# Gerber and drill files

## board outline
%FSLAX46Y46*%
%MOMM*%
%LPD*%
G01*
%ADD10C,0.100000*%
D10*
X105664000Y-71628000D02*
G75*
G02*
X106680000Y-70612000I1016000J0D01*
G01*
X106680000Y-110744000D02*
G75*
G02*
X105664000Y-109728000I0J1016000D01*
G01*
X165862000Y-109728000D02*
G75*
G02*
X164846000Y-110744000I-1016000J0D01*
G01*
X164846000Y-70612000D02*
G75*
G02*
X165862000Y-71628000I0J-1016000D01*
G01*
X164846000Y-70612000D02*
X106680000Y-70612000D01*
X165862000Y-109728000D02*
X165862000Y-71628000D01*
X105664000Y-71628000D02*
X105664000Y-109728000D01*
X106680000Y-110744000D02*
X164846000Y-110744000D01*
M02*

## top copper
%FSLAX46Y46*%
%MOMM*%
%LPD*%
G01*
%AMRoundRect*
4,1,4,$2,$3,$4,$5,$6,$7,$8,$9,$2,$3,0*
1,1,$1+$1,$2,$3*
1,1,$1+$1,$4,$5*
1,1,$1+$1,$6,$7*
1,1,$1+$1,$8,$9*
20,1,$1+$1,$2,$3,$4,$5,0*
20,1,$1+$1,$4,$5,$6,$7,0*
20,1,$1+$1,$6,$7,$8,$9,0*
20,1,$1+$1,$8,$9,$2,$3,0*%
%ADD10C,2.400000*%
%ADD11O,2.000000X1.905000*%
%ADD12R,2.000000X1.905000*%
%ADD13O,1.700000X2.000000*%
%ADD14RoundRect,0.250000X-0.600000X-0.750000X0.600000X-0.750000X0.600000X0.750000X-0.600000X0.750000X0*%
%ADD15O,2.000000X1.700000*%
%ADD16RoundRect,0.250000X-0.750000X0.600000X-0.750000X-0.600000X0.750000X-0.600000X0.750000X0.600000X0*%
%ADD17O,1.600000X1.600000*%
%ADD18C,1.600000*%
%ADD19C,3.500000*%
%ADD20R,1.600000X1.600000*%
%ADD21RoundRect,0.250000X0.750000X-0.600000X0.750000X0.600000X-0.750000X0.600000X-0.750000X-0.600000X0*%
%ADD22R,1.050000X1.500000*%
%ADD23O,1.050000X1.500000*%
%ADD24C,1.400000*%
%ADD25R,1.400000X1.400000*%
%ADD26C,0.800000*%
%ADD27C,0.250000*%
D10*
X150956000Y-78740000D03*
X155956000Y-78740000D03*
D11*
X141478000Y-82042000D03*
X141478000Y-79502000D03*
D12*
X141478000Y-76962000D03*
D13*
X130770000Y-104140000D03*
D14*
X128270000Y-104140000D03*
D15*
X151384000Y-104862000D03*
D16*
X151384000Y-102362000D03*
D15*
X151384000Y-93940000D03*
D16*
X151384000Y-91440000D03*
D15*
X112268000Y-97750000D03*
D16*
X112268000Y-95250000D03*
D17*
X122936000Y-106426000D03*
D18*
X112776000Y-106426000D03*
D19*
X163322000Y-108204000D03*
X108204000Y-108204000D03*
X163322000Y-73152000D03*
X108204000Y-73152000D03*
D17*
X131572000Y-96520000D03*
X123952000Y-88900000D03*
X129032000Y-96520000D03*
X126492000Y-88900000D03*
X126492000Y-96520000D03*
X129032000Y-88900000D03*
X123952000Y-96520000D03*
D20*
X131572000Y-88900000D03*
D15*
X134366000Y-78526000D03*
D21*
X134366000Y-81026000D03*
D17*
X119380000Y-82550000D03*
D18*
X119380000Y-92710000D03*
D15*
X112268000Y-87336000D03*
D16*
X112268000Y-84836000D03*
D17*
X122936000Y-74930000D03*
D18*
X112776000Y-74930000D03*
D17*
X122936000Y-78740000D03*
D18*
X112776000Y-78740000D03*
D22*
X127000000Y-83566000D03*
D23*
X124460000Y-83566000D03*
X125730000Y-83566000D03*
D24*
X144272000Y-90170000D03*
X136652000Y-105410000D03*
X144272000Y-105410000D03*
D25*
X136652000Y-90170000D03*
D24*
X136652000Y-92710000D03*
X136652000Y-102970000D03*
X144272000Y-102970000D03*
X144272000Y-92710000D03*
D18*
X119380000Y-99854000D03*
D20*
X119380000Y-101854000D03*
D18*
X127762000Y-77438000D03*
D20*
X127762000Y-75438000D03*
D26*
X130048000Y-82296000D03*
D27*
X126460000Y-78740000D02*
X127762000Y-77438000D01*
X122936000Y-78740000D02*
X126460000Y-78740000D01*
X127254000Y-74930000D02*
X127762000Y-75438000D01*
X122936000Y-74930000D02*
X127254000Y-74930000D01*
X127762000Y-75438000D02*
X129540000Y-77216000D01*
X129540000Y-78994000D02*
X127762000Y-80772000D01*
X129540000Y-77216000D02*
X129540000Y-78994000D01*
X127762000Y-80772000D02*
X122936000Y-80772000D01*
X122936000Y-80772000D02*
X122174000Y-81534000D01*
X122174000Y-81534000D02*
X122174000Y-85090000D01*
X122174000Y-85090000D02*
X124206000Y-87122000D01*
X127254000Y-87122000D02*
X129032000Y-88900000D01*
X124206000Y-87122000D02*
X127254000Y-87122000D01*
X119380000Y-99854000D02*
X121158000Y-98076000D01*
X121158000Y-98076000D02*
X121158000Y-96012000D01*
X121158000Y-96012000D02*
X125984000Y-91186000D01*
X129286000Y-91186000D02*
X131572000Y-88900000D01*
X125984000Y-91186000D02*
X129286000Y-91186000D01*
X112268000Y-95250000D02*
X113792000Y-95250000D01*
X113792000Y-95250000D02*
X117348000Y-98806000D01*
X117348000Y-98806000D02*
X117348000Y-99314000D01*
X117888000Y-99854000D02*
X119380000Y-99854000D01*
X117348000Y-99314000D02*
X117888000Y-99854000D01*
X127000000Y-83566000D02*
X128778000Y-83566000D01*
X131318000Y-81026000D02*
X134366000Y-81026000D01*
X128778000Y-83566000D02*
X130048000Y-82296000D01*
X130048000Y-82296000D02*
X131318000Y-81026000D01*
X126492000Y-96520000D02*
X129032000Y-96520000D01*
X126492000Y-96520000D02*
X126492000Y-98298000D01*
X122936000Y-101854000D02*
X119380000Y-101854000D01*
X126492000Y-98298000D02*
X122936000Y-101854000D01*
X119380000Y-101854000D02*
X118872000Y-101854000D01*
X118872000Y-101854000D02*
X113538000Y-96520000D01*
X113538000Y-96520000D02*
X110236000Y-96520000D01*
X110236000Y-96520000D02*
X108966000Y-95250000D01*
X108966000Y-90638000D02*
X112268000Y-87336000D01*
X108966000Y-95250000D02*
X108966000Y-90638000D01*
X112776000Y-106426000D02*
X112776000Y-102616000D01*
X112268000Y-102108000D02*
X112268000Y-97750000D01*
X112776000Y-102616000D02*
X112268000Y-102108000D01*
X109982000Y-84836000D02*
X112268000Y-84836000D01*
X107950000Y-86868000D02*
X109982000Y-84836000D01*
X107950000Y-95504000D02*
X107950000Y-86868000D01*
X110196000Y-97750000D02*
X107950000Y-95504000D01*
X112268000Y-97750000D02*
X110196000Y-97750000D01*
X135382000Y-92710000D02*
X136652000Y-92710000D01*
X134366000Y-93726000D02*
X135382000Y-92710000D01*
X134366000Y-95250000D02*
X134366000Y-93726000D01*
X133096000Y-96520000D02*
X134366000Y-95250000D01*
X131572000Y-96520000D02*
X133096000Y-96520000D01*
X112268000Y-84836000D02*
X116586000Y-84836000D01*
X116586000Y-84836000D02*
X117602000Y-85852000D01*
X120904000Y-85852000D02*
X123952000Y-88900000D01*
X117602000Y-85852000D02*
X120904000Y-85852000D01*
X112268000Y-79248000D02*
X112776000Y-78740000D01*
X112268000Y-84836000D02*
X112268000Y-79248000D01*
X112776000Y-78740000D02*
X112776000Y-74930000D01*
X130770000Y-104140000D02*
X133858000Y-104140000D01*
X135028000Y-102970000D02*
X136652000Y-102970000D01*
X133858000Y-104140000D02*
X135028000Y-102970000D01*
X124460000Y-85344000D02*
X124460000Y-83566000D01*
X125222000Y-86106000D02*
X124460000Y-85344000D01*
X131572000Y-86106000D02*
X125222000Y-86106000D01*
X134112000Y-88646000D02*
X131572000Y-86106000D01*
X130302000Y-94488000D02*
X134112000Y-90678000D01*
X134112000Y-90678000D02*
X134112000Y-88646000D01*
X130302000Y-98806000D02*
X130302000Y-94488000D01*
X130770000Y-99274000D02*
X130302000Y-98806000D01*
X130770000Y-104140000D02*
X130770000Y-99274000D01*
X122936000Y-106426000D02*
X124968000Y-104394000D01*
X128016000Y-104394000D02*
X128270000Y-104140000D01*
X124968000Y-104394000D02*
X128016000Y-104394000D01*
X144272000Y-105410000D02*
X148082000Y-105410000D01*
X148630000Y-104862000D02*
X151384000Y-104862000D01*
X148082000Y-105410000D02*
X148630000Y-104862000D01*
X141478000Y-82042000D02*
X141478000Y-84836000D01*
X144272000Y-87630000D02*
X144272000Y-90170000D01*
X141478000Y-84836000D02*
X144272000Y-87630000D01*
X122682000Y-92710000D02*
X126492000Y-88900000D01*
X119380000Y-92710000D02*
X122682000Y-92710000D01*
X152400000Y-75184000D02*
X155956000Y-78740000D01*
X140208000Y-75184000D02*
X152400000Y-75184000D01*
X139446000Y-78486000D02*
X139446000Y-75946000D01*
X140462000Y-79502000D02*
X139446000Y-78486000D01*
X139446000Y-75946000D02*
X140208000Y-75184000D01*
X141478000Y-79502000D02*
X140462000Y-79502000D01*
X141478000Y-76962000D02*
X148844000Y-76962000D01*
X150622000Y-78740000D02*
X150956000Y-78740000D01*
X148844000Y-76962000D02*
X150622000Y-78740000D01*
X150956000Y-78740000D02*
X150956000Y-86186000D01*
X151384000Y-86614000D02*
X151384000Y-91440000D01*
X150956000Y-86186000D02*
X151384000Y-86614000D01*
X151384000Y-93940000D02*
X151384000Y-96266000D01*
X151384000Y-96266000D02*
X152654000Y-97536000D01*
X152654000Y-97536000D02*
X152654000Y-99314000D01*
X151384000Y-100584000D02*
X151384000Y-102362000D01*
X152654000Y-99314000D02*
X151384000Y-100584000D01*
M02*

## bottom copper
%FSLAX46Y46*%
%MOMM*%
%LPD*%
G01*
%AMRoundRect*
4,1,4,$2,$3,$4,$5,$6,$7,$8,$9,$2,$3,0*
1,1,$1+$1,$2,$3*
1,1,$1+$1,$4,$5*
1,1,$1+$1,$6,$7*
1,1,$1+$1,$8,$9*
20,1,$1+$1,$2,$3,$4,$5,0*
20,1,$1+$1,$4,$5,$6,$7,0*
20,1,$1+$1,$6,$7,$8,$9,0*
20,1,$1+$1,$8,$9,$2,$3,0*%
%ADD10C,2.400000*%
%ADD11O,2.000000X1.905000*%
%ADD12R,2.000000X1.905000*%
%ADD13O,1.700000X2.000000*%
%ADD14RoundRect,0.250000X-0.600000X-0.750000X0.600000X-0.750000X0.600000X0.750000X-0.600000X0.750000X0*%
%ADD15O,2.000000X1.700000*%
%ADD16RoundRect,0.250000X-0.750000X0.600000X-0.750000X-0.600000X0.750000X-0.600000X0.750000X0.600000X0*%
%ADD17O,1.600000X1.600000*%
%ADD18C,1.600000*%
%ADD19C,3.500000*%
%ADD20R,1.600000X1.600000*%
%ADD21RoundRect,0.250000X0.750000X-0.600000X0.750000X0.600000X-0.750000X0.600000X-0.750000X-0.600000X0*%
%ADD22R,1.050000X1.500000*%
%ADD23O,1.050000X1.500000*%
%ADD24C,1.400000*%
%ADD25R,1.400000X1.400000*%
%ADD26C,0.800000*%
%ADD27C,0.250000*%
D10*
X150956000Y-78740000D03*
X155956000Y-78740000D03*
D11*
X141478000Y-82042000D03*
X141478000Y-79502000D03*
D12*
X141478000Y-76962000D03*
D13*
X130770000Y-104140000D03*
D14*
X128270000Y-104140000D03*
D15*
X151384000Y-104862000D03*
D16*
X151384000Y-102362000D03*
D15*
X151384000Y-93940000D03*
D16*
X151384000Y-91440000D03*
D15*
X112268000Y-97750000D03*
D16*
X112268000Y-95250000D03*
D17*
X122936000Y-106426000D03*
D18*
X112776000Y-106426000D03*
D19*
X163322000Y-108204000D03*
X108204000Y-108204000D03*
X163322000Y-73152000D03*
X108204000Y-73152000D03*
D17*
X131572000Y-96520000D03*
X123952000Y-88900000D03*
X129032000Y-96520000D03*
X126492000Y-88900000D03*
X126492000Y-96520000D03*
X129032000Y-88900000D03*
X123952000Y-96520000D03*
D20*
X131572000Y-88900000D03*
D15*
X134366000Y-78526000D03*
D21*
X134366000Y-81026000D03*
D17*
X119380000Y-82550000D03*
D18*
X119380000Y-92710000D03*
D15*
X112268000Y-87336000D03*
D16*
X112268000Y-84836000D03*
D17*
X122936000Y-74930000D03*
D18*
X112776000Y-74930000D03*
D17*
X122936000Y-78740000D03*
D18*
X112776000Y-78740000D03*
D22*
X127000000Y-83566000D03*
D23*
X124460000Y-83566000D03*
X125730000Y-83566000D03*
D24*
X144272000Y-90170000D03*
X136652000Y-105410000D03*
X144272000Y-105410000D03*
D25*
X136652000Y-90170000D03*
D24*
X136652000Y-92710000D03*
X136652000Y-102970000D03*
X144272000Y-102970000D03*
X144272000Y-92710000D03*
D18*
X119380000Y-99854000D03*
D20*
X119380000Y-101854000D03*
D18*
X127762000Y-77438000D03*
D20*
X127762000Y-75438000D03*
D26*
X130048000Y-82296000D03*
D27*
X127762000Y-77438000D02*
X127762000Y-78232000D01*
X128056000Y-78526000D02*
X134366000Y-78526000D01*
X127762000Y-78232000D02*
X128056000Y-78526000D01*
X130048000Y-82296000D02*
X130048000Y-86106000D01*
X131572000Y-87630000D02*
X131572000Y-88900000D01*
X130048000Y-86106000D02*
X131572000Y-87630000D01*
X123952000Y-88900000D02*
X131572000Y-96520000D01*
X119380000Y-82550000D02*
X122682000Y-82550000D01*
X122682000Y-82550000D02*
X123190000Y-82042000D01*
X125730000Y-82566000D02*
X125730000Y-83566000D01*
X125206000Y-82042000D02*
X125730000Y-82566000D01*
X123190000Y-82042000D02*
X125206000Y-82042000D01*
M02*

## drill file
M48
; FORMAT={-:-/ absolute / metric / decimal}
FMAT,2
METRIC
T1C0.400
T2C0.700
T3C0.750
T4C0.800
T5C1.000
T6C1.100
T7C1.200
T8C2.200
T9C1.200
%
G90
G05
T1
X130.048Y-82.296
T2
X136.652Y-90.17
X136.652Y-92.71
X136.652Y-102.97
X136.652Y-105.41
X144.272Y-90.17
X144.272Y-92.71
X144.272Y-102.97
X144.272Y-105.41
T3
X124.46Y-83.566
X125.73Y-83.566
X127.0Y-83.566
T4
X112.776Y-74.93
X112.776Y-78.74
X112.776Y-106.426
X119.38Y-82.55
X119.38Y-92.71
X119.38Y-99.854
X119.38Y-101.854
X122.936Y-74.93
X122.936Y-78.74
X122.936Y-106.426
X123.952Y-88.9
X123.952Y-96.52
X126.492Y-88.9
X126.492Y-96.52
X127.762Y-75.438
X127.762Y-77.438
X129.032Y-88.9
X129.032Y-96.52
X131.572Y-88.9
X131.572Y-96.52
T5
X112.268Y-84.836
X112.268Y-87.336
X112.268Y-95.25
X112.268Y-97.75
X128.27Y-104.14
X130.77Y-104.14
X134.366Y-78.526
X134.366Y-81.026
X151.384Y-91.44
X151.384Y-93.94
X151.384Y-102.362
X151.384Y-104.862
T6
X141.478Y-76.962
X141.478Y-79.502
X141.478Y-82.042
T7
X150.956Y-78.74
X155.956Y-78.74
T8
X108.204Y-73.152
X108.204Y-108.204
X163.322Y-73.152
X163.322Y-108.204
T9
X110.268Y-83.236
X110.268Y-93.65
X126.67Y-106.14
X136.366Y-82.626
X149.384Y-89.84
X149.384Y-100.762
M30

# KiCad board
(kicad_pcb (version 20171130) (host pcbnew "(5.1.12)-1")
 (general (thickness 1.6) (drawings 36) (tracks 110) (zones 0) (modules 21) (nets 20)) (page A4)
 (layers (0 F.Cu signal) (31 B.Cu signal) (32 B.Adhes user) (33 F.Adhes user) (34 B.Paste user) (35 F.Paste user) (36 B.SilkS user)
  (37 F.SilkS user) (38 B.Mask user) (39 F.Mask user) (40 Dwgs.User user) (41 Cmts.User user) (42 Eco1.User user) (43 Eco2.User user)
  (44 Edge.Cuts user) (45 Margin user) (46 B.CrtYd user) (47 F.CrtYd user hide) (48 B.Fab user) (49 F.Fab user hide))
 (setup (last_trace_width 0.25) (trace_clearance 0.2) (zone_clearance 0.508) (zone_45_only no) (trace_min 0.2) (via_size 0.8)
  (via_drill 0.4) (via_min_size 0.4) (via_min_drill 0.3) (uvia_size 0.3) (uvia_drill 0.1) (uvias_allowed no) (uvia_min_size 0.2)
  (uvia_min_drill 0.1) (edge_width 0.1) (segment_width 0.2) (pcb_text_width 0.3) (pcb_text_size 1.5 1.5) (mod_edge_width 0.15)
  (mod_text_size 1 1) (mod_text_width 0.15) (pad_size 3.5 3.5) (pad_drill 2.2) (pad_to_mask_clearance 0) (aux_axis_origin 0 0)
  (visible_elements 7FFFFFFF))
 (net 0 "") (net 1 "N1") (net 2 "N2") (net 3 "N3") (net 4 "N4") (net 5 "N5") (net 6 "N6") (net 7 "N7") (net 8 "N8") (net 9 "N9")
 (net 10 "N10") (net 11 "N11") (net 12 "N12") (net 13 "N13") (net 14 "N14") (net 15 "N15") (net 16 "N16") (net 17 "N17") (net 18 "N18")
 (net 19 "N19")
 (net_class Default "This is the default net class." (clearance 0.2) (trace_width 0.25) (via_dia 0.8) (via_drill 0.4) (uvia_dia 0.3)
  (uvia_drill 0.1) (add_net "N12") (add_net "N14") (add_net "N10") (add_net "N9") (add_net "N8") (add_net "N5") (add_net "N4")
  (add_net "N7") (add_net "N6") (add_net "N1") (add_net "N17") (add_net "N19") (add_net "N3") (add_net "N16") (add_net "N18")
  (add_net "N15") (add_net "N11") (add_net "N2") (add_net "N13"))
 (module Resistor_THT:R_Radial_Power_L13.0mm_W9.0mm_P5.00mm (layer F.Cu) (at 155.956 78.74 180)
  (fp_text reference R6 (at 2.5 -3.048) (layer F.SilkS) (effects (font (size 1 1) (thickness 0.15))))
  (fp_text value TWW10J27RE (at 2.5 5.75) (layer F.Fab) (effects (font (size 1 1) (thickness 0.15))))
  (pad 2 thru_hole circle (at 5 0 180) (size 2.4 2.4) (drill 1.2) (layers *.Cu *.Mask) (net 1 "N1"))
  (pad 1 thru_hole circle (at 0 0 180) (size 2.4 2.4) (drill 1.2) (layers *.Cu *.Mask) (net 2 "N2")))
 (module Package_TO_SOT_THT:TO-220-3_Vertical (layer F.Cu) (at 141.478 76.962 270)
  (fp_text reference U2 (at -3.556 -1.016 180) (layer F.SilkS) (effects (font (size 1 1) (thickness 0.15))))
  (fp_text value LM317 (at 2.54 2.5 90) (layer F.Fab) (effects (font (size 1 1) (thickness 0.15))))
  (pad 3 thru_hole oval (at 5.08 0 270) (size 1.905 2) (drill 1.1) (layers *.Cu *.Mask) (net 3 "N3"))
  (pad 2 thru_hole oval (at 2.54 0 270) (size 1.905 2) (drill 1.1) (layers *.Cu *.Mask) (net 2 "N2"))
  (pad 1 thru_hole rect (at 0 0 270) (size 1.905 2) (drill 1.1) (layers *.Cu *.Mask) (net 1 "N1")))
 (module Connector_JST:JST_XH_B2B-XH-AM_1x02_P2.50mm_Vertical (layer F.Cu) (at 128.27 104.14)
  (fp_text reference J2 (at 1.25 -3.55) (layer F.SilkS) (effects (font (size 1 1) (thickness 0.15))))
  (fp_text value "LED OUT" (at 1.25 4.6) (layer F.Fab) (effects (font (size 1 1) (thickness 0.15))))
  (pad "" np_thru_hole circle (at -1.6 2) (size 1.2 1.2) (drill 1.2) (layers *.Cu *.Mask))
  (pad 2 thru_hole oval (at 2.5 0) (size 1.7 2) (drill 1) (layers *.Cu *.Mask) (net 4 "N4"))
  (pad 1 thru_hole roundrect (at 0 0) (size 1.7 2) (drill 1) (layers *.Cu *.Mask) (roundrect_rratio 0.147059) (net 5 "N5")))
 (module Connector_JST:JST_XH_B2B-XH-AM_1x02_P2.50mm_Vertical (layer F.Cu) (at 151.384 102.362 270)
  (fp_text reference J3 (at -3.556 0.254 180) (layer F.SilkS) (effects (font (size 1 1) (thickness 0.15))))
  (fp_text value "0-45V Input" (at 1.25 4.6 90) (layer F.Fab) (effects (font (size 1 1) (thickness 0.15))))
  (pad "" np_thru_hole circle (at -1.6 2 270) (size 1.2 1.2) (drill 1.2) (layers *.Cu *.Mask))
  (pad 2 thru_hole oval (at 2.5 0 270) (size 1.7 2) (drill 1) (layers *.Cu *.Mask) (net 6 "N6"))
  (pad 1 thru_hole roundrect (at 0 0 270) (size 1.7 2) (drill 1) (layers *.Cu *.Mask) (roundrect_rratio 0.147059) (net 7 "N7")))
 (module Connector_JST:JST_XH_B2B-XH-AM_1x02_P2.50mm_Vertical (layer F.Cu) (at 151.384 91.44 270)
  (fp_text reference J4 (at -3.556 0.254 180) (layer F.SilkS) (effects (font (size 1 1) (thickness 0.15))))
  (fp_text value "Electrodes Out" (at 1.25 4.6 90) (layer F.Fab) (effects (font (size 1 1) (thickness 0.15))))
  (pad "" np_thru_hole circle (at -1.6 2 270) (size 1.2 1.2) (drill 1.2) (layers *.Cu *.Mask))
  (pad 2 thru_hole oval (at 2.5 0 270) (size 1.7 2) (drill 1) (layers *.Cu *.Mask) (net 7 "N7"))
  (pad 1 thru_hole roundrect (at 0 0 270) (size 1.7 2) (drill 1) (layers *.Cu *.Mask) (roundrect_rratio 0.147059) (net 1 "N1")))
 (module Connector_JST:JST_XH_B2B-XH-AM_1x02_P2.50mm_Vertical (layer F.Cu) (at 112.268 95.25 270)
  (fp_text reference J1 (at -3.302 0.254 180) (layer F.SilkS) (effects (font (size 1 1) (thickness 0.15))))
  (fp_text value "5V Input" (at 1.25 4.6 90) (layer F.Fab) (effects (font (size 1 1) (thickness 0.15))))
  (pad "" np_thru_hole circle (at -1.6 2 270) (size 1.2 1.2) (drill 1.2) (layers *.Cu *.Mask))
  (pad 2 thru_hole oval (at 2.5 0 270) (size 1.7 2) (drill 1) (layers *.Cu *.Mask) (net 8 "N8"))
  (pad 1 thru_hole roundrect (at 0 0 270) (size 1.7 2) (drill 1) (layers *.Cu *.Mask) (roundrect_rratio 0.147059) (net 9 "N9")))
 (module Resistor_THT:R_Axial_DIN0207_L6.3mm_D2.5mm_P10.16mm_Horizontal (layer F.Cu) (at 112.776 106.426)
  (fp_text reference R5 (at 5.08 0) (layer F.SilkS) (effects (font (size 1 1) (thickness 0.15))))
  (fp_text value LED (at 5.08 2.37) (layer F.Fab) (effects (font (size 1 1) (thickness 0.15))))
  (pad 2 thru_hole oval (at 10.16 0) (size 1.6 1.6) (drill 0.8) (layers *.Cu *.Mask) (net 5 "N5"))
  (pad 1 thru_hole circle (at 0 0) (size 1.6 1.6) (drill 0.8) (layers *.Cu *.Mask) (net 8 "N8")))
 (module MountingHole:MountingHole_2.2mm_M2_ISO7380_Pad (layer F.Cu) (at 163.322 108.204)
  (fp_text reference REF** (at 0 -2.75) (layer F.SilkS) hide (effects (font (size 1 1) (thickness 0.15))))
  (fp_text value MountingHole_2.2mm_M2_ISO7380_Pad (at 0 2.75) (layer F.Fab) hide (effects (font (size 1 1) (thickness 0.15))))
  (pad 1 thru_hole circle (at 0 0) (size 3.5 3.5) (drill 2.2) (layers *.Cu *.Mask)))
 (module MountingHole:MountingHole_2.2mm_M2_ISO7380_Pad (layer F.Cu) (at 108.204 108.204)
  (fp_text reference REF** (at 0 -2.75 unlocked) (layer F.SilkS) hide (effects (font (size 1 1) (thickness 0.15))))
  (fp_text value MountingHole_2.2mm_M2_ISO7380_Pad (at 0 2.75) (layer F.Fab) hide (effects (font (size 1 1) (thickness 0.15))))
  (pad 1 thru_hole circle (at 0 0) (size 3.5 3.5) (drill 2.2) (layers *.Cu *.Mask)))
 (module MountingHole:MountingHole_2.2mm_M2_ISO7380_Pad (layer F.Cu) (at 163.322 73.152)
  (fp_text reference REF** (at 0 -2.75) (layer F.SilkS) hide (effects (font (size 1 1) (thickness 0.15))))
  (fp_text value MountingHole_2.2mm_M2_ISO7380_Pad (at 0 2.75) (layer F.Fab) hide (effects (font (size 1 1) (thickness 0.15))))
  (pad 1 thru_hole circle (at 0 0) (size 3.5 3.5) (drill 2.2) (layers *.Cu *.Mask)))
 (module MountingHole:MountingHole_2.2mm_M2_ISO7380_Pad (layer F.Cu) (at 108.204 73.152)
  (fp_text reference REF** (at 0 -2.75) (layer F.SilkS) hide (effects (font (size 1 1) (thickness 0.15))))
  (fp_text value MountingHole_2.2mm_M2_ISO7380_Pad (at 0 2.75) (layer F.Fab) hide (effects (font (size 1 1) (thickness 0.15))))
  (pad 1 thru_hole circle (at 0 0) (size 3.5 3.5) (drill 2.2) (layers *.Cu *.Mask)))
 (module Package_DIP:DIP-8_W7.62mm (layer F.Cu) (at 131.572 88.9 270)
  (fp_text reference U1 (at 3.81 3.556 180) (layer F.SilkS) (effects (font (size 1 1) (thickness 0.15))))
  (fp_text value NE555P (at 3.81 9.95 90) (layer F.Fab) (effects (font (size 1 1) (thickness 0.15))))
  (pad 8 thru_hole oval (at 7.62 0 270) (size 1.6 1.6) (drill 0.8) (layers *.Cu *.Mask) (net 8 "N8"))
  (pad 4 thru_hole oval (at 0 7.62 270) (size 1.6 1.6) (drill 0.8) (layers *.Cu *.Mask) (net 8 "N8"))
  (pad 7 thru_hole oval (at 7.62 2.54 270) (size 1.6 1.6) (drill 0.8) (layers *.Cu *.Mask) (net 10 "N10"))
  (pad 3 thru_hole oval (at 0 5.08 270) (size 1.6 1.6) (drill 0.8) (layers *.Cu *.Mask) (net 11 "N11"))
  (pad 6 thru_hole oval (at 7.62 5.08 270) (size 1.6 1.6) (drill 0.8) (layers *.Cu *.Mask) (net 10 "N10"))
  (pad 2 thru_hole oval (at 0 2.54 270) (size 1.6 1.6) (drill 0.8) (layers *.Cu *.Mask) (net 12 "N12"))
  (pad 5 thru_hole oval (at 7.62 7.62 270) (size 1.6 1.6) (drill 0.8) (layers *.Cu *.Mask) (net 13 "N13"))
  (pad 1 thru_hole rect (at 0 0 270) (size 1.6 1.6) (drill 0.8) (layers *.Cu *.Mask) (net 9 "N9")))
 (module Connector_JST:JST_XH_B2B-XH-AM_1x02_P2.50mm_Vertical (layer F.Cu) (at 134.366 81.026 90)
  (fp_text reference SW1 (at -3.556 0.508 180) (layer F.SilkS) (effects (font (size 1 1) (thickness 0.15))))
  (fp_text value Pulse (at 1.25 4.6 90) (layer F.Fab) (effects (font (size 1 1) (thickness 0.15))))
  (pad "" np_thru_hole circle (at -1.6 2 90) (size 1.2 1.2) (drill 1.2) (layers *.Cu *.Mask))
  (pad 2 thru_hole oval (at 2.5 0 90) (size 1.7 2) (drill 1) (layers *.Cu *.Mask) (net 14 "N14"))
  (pad 1 thru_hole roundrect (at 0 0 90) (size 1.7 2) (drill 1) (layers *.Cu *.Mask) (roundrect_rratio 0.147059) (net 9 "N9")))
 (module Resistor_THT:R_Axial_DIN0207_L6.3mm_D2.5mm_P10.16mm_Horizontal (layer F.Cu) (at 119.38 92.71 90)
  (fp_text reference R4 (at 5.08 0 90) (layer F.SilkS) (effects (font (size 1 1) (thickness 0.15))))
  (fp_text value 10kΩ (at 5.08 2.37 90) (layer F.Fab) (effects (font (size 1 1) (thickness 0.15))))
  (pad 2 thru_hole oval (at 10.16 0 90) (size 1.6 1.6) (drill 0.8) (layers *.Cu *.Mask) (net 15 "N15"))
  (pad 1 thru_hole circle (at 0 0 90) (size 1.6 1.6) (drill 0.8) (layers *.Cu *.Mask) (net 11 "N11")))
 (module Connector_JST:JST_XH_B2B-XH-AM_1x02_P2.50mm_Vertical (layer F.Cu) (at 112.268 84.836 270)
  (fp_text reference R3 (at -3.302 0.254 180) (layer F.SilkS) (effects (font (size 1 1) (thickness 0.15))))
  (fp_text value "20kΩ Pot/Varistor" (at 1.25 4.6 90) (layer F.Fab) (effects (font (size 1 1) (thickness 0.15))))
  (pad "" np_thru_hole circle (at -1.6 2 270) (size 1.2 1.2) (drill 1.2) (layers *.Cu *.Mask))
  (pad 2 thru_hole oval (at 2.5 0 270) (size 1.7 2) (drill 1) (layers *.Cu *.Mask) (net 10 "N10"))
  (pad 1 thru_hole roundrect (at 0 0 270) (size 1.7 2) (drill 1) (layers *.Cu *.Mask) (roundrect_rratio 0.147059) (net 8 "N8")))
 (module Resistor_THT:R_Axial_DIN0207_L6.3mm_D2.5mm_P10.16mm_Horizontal (layer F.Cu) (at 112.776 74.93)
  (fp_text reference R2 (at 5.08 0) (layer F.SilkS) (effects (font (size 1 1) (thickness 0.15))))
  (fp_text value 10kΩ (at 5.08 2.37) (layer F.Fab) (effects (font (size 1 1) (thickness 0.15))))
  (pad 2 thru_hole oval (at 10.16 0) (size 1.6 1.6) (drill 0.8) (layers *.Cu *.Mask) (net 12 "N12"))
  (pad 1 thru_hole circle (at 0 0) (size 1.6 1.6) (drill 0.8) (layers *.Cu *.Mask) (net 8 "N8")))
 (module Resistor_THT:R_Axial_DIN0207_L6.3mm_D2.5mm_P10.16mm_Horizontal (layer F.Cu) (at 112.776 78.74)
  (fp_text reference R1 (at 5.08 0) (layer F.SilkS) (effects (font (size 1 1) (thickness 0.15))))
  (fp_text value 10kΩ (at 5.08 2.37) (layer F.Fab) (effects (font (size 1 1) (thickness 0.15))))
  (pad 2 thru_hole oval (at 10.16 0) (size 1.6 1.6) (drill 0.8) (layers *.Cu *.Mask) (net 14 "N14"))
  (pad 1 thru_hole circle (at 0 0) (size 1.6 1.6) (drill 0.8) (layers *.Cu *.Mask) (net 8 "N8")))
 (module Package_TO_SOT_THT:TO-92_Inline (layer F.Cu) (at 127 83.566 180)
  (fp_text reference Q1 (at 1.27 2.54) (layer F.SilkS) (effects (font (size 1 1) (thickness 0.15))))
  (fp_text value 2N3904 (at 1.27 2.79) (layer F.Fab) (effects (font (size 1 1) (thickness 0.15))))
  (pad 1 thru_hole rect (at 0 0 180) (size 1.05 1.5) (drill 0.75) (layers *.Cu *.Mask) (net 9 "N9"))
  (pad 3 thru_hole oval (at 2.54 0 180) (size 1.05 1.5) (drill 0.75) (layers *.Cu *.Mask) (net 4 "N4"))
  (pad 2 thru_hole oval (at 1.27 0 180) (size 1.05 1.5) (drill 0.75) (layers *.Cu *.Mask) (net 15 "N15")))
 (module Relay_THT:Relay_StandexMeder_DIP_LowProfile (layer F.Cu) (at 136.652 90.17)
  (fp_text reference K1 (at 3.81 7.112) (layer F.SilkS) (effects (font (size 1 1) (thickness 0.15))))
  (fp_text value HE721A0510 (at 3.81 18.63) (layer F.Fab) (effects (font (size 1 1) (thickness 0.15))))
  (pad 14 thru_hole circle (at 7.62 0) (size 1.4 1.4) (drill 0.7) (layers *.Cu *.Mask) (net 3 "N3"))
  (pad 7 thru_hole circle (at 0 15.24) (size 1.4 1.4) (drill 0.7) (layers *.Cu *.Mask) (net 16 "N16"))
  (pad 8 thru_hole circle (at 7.62 15.24) (size 1.4 1.4) (drill 0.7) (layers *.Cu *.Mask) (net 6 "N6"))
  (pad 1 thru_hole rect (at 0 0) (size 1.4 1.4) (drill 0.7) (layers *.Cu *.Mask) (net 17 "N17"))
  (pad 2 thru_hole circle (at 0 2.54) (size 1.4 1.4) (drill 0.7) (layers *.Cu *.Mask) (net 8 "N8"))
  (pad 6 thru_hole circle (at 0 12.8) (size 1.4 1.4) (drill 0.7) (layers *.Cu *.Mask) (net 4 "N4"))
  (pad 9 thru_hole circle (at 7.62 12.8) (size 1.4 1.4) (drill 0.7) (layers *.Cu *.Mask) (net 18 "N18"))
  (pad 13 thru_hole circle (at 7.62 2.54) (size 1.4 1.4) (drill 0.7) (layers *.Cu *.Mask) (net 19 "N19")))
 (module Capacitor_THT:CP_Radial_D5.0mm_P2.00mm (layer F.Cu) (at 119.38 101.854 90)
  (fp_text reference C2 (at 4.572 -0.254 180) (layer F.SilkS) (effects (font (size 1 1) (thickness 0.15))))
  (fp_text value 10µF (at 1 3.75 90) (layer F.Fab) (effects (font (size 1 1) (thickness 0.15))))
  (pad 2 thru_hole circle (at 2 0 90) (size 1.6 1.6) (drill 0.8) (layers *.Cu *.Mask) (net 9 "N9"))
  (pad 1 thru_hole rect (at 0 0 90) (size 1.6 1.6) (drill 0.8) (layers *.Cu *.Mask) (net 10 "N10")))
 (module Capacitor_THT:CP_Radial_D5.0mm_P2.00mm (layer F.Cu) (at 127.762 75.438 270)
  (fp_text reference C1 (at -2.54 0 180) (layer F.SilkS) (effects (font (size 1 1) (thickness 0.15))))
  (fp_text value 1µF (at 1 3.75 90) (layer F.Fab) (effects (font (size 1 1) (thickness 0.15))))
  (pad 2 thru_hole circle (at 2 0 270) (size 1.6 1.6) (drill 0.8) (layers *.Cu *.Mask) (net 14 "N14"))
  (pad 1 thru_hole rect (at 0 0 270) (size 1.6 1.6) (drill 0.8) (layers *.Cu *.Mask) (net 12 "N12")))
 (gr_arc (start 106.68 71.628) (end 106.68 70.612) (angle -90) (layer Edge.Cuts) (width 0.1))
 (gr_arc (start 106.68 109.728) (end 105.664 109.728) (angle -90) (layer Edge.Cuts) (width 0.1))
 (gr_arc (start 164.846 109.728) (end 164.846 110.744) (angle -90) (layer Edge.Cuts) (width 0.1))
 (gr_arc (start 164.846 71.628) (end 165.862 71.628) (angle -90) (layer Edge.Cuts) (width 0.1))
 (gr_line (start 164.846 70.612) (end 106.68 70.612) (layer Edge.Cuts) (width 0.1))
 (gr_line (start 165.862 109.728) (end 165.862 71.628) (layer Edge.Cuts) (width 0.1))
 (gr_line (start 105.664 71.628) (end 105.664 109.728) (layer Edge.Cuts) (width 0.1))
 (gr_line (start 106.68 110.744) (end 164.846 110.744) (layer Edge.Cuts) (width 0.1))
 (segment (start 126.46 78.74) (end 127.762 77.438) (width 0.25) (layer F.Cu) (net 14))
 (segment (start 122.936 78.74) (end 126.46 78.74) (width 0.25) (layer F.Cu) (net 14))
 (segment (start 127.762 77.438) (end 127.762 78.232) (width 0.25) (layer B.Cu) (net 14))
 (segment (start 128.056 78.526) (end 134.366 78.526) (width 0.25) (layer B.Cu) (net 14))
 (segment (start 127.762 78.232) (end 128.056 78.526) (width 0.25) (layer B.Cu) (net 14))
 (segment (start 127.254 74.93) (end 127.762 75.438) (width 0.25) (layer F.Cu) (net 12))
 (segment (start 122.936 74.93) (end 127.254 74.93) (width 0.25) (layer F.Cu) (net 12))
 (segment (start 127.762 75.438) (end 129.54 77.216) (width 0.25) (layer F.Cu) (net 12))
 (segment (start 129.54 78.994) (end 127.762 80.772) (width 0.25) (layer F.Cu) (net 12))
 (segment (start 129.54 77.216) (end 129.54 78.994) (width 0.25) (layer F.Cu) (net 12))
 (segment (start 127.762 80.772) (end 122.936 80.772) (width 0.25) (layer F.Cu) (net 12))
 (segment (start 122.936 80.772) (end 122.174 81.534) (width 0.25) (layer F.Cu) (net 12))
 (segment (start 122.174 81.534) (end 122.174 85.09) (width 0.25) (layer F.Cu) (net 12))
 (segment (start 122.174 85.09) (end 124.206 87.122) (width 0.25) (layer F.Cu) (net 12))
 (segment (start 127.254 87.122) (end 129.032 88.9) (width 0.25) (layer F.Cu) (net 12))
 (segment (start 124.206 87.122) (end 127.254 87.122) (width 0.25) (layer F.Cu) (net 12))
 (segment (start 119.38 99.854) (end 121.158 98.076) (width 0.25) (layer F.Cu) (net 9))
 (segment (start 121.158 98.076) (end 121.158 96.012) (width 0.25) (layer F.Cu) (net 9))
 (segment (start 121.158 96.012) (end 125.984 91.186) (width 0.25) (layer F.Cu) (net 9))
 (segment (start 129.286 91.186) (end 131.572 88.9) (width 0.25) (layer F.Cu) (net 9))
 (segment (start 125.984 91.186) (end 129.286 91.186) (width 0.25) (layer F.Cu) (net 9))
 (segment (start 112.268 95.25) (end 113.792 95.25) (width 0.25) (layer F.Cu) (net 9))
 (segment (start 113.792 95.25) (end 117.348 98.806) (width 0.25) (layer F.Cu) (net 9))
 (segment (start 117.348 98.806) (end 117.348 99.314) (width 0.25) (layer F.Cu) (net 9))
 (segment (start 117.888 99.854) (end 119.38 99.854) (width 0.25) (layer F.Cu) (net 9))
 (segment (start 117.348 99.314) (end 117.888 99.854) (width 0.25) (layer F.Cu) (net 9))
 (segment (start 127 83.566) (end 128.778 83.566) (width 0.25) (layer F.Cu) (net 9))
 (segment (start 131.318 81.026) (end 134.366 81.026) (width 0.25) (layer F.Cu) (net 9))
 (segment (start 128.778 83.566) (end 130.048 82.296) (width 0.25) (layer F.Cu) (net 9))
 (segment (start 130.048 82.296) (end 131.318 81.026) (width 0.25) (layer F.Cu) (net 9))
 (via (at 130.048 82.296) (size 0.8) (drill 0.4) (layers F.Cu B.Cu) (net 9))
 (segment (start 130.048 82.296) (end 130.048 86.106) (width 0.25) (layer B.Cu) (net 9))
 (segment (start 131.572 87.63) (end 131.572 88.9) (width 0.25) (layer B.Cu) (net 9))
 (segment (start 130.048 86.106) (end 131.572 87.63) (width 0.25) (layer B.Cu) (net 9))
 (segment (start 126.492 96.52) (end 129.032 96.52) (width 0.25) (layer F.Cu) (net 10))
 (segment (start 126.492 96.52) (end 126.492 98.298) (width 0.25) (layer F.Cu) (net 10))
 (segment (start 122.936 101.854) (end 119.38 101.854) (width 0.25) (layer F.Cu) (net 10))
 (segment (start 126.492 98.298) (end 122.936 101.854) (width 0.25) (layer F.Cu) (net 10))
 (segment (start 119.38 101.854) (end 118.872 101.854) (width 0.25) (layer F.Cu) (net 10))
 (segment (start 118.872 101.854) (end 113.538 96.52) (width 0.25) (layer F.Cu) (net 10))
 (segment (start 113.538 96.52) (end 110.236 96.52) (width 0.25) (layer F.Cu) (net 10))
 (segment (start 110.236 96.52) (end 108.966 95.25) (width 0.25) (layer F.Cu) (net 10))
 (segment (start 108.966 90.638) (end 112.268 87.336) (width 0.25) (layer F.Cu) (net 10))
 (segment (start 108.966 95.25) (end 108.966 90.638) (width 0.25) (layer F.Cu) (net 10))
 (segment (start 112.776 106.426) (end 112.776 102.616) (width 0.25) (layer F.Cu) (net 8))
 (segment (start 112.268 102.108) (end 112.268 97.75) (width 0.25) (layer F.Cu) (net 8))
 (segment (start 112.776 102.616) (end 112.268 102.108) (width 0.25) (layer F.Cu) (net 8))
 (segment (start 109.982 84.836) (end 112.268 84.836) (width 0.25) (layer F.Cu) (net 8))
 (segment (start 107.95 86.868) (end 109.982 84.836) (width 0.25) (layer F.Cu) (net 8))
 (segment (start 107.95 95.504) (end 107.95 86.868) (width 0.25) (layer F.Cu) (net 8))
 (segment (start 110.196 97.75) (end 107.95 95.504) (width 0.25) (layer F.Cu) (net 8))
 (segment (start 112.268 97.75) (end 110.196 97.75) (width 0.25) (layer F.Cu) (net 8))
 (segment (start 135.382 92.71) (end 136.652 92.71) (width 0.25) (layer F.Cu) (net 8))
 (segment (start 134.366 93.726) (end 135.382 92.71) (width 0.25) (layer F.Cu) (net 8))
 (segment (start 134.366 95.25) (end 134.366 93.726) (width 0.25) (layer F.Cu) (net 8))
 (segment (start 133.096 96.52) (end 134.366 95.25) (width 0.25) (layer F.Cu) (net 8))
 (segment (start 131.572 96.52) (end 133.096 96.52) (width 0.25) (layer F.Cu) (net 8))
 (segment (start 112.268 84.836) (end 116.586 84.836) (width 0.25) (layer F.Cu) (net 8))
 (segment (start 116.586 84.836) (end 117.602 85.852) (width 0.25) (layer F.Cu) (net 8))
 (segment (start 120.904 85.852) (end 123.952 88.9) (width 0.25) (layer F.Cu) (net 8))
 (segment (start 117.602 85.852) (end 120.904 85.852) (width 0.25) (layer F.Cu) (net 8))
 (segment (start 112.268 79.248) (end 112.776 78.74) (width 0.25) (layer F.Cu) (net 8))
 (segment (start 112.268 84.836) (end 112.268 79.248) (width 0.25) (layer F.Cu) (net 8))
 (segment (start 112.776 78.74) (end 112.776 74.93) (width 0.25) (layer F.Cu) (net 8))
 (segment (start 123.952 88.9) (end 131.572 96.52) (width 0.25) (layer B.Cu) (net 8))
 (segment (start 130.77 104.14) (end 133.858 104.14) (width 0.25) (layer F.Cu) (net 4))
 (segment (start 135.028 102.97) (end 136.652 102.97) (width 0.25) (layer F.Cu) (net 4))
 (segment (start 133.858 104.14) (end 135.028 102.97) (width 0.25) (layer F.Cu) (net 4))
 (segment (start 124.46 85.344) (end 124.46 83.566) (width 0.25) (layer F.Cu) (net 4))
 (segment (start 125.222 86.106) (end 124.46 85.344) (width 0.25) (layer F.Cu) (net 4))
 (segment (start 131.572 86.106) (end 125.222 86.106) (width 0.25) (layer F.Cu) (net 4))
 (segment (start 134.112 88.646) (end 131.572 86.106) (width 0.25) (layer F.Cu) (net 4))
 (segment (start 130.302 94.488) (end 134.112 90.678) (width 0.25) (layer F.Cu) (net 4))
 (segment (start 134.112 90.678) (end 134.112 88.646) (width 0.25) (layer F.Cu) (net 4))
 (segment (start 130.302 98.806) (end 130.302 94.488) (width 0.25) (layer F.Cu) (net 4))
 (segment (start 130.77 99.274) (end 130.302 98.806) (width 0.25) (layer F.Cu) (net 4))
 (segment (start 130.77 104.14) (end 130.77 99.274) (width 0.25) (layer F.Cu) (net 4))
 (segment (start 122.936 106.426) (end 124.968 104.394) (width 0.25) (layer F.Cu) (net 5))
 (segment (start 128.016 104.394) (end 128.27 104.14) (width 0.25) (layer F.Cu) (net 5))
 (segment (start 124.968 104.394) (end 128.016 104.394) (width 0.25) (layer F.Cu) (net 5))
 (segment (start 144.272 105.41) (end 148.082 105.41) (width 0.25) (layer F.Cu) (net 6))
 (segment (start 148.63 104.862) (end 151.384 104.862) (width 0.25) (layer F.Cu) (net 6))
 (segment (start 148.082 105.41) (end 148.63 104.862) (width 0.25) (layer F.Cu) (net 6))
 (segment (start 141.478 82.042) (end 141.478 84.836) (width 0.25) (layer F.Cu) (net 3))
 (segment (start 144.272 87.63) (end 144.272 90.17) (width 0.25) (layer F.Cu) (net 3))
 (segment (start 141.478 84.836) (end 144.272 87.63) (width 0.25) (layer F.Cu) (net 3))
 (segment (start 119.38 82.55) (end 122.682 82.55) (width 0.25) (layer B.Cu) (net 15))
 (segment (start 122.682 82.55) (end 123.19 82.042) (width 0.25) (layer B.Cu) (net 15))
 (segment (start 125.73 82.566) (end 125.73 83.566) (width 0.25) (layer B.Cu) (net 15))
 (segment (start 125.206 82.042) (end 125.73 82.566) (width 0.25) (layer B.Cu) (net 15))
 (segment (start 123.19 82.042) (end 125.206 82.042) (width 0.25) (layer B.Cu) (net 15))
 (segment (start 122.682 92.71) (end 126.492 88.9) (width 0.25) (layer F.Cu) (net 11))
 (segment (start 119.38 92.71) (end 122.682 92.71) (width 0.25) (layer F.Cu) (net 11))
 (segment (start 152.4 75.184) (end 155.956 78.74) (width 0.25) (layer F.Cu) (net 2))
 (segment (start 140.208 75.184) (end 152.4 75.184) (width 0.25) (layer F.Cu) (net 2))
 (segment (start 139.446 78.486) (end 139.446 75.946) (width 0.25) (layer F.Cu) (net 2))
 (segment (start 140.462 79.502) (end 139.446 78.486) (width 0.25) (layer F.Cu) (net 2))
 (segment (start 139.446 75.946) (end 140.208 75.184) (width 0.25) (layer F.Cu) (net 2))
 (segment (start 141.478 79.502) (end 140.462 79.502) (width 0.25) (layer F.Cu) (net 2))
 (segment (start 141.478 76.962) (end 148.844 76.962) (width 0.25) (layer F.Cu) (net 1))
 (segment (start 150.622 78.74) (end 150.956 78.74) (width 0.25) (layer F.Cu) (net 1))
 (segment (start 148.844 76.962) (end 150.622 78.74) (width 0.25) (layer F.Cu) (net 1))
 (segment (start 150.956 78.74) (end 150.956 86.186) (width 0.25) (layer F.Cu) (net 1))
 (segment (start 151.384 86.614) (end 151.384 91.44) (width 0.25) (layer F.Cu) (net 1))
 (segment (start 150.956 86.186) (end 151.384 86.614) (width 0.25) (layer F.Cu) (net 1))
 (segment (start 151.384 93.94) (end 151.384 96.266) (width 0.25) (layer F.Cu) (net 7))
 (segment (start 151.384 96.266) (end 152.654 97.536) (width 0.25) (layer F.Cu) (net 7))
 (segment (start 152.654 97.536) (end 152.654 99.314) (width 0.25) (layer F.Cu) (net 7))
 (segment (start 151.384 100.584) (end 151.384 102.362) (width 0.25) (layer F.Cu) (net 7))
 (segment (start 152.654 99.314) (end 151.384 100.584) (width 0.25) (layer F.Cu) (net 7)))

